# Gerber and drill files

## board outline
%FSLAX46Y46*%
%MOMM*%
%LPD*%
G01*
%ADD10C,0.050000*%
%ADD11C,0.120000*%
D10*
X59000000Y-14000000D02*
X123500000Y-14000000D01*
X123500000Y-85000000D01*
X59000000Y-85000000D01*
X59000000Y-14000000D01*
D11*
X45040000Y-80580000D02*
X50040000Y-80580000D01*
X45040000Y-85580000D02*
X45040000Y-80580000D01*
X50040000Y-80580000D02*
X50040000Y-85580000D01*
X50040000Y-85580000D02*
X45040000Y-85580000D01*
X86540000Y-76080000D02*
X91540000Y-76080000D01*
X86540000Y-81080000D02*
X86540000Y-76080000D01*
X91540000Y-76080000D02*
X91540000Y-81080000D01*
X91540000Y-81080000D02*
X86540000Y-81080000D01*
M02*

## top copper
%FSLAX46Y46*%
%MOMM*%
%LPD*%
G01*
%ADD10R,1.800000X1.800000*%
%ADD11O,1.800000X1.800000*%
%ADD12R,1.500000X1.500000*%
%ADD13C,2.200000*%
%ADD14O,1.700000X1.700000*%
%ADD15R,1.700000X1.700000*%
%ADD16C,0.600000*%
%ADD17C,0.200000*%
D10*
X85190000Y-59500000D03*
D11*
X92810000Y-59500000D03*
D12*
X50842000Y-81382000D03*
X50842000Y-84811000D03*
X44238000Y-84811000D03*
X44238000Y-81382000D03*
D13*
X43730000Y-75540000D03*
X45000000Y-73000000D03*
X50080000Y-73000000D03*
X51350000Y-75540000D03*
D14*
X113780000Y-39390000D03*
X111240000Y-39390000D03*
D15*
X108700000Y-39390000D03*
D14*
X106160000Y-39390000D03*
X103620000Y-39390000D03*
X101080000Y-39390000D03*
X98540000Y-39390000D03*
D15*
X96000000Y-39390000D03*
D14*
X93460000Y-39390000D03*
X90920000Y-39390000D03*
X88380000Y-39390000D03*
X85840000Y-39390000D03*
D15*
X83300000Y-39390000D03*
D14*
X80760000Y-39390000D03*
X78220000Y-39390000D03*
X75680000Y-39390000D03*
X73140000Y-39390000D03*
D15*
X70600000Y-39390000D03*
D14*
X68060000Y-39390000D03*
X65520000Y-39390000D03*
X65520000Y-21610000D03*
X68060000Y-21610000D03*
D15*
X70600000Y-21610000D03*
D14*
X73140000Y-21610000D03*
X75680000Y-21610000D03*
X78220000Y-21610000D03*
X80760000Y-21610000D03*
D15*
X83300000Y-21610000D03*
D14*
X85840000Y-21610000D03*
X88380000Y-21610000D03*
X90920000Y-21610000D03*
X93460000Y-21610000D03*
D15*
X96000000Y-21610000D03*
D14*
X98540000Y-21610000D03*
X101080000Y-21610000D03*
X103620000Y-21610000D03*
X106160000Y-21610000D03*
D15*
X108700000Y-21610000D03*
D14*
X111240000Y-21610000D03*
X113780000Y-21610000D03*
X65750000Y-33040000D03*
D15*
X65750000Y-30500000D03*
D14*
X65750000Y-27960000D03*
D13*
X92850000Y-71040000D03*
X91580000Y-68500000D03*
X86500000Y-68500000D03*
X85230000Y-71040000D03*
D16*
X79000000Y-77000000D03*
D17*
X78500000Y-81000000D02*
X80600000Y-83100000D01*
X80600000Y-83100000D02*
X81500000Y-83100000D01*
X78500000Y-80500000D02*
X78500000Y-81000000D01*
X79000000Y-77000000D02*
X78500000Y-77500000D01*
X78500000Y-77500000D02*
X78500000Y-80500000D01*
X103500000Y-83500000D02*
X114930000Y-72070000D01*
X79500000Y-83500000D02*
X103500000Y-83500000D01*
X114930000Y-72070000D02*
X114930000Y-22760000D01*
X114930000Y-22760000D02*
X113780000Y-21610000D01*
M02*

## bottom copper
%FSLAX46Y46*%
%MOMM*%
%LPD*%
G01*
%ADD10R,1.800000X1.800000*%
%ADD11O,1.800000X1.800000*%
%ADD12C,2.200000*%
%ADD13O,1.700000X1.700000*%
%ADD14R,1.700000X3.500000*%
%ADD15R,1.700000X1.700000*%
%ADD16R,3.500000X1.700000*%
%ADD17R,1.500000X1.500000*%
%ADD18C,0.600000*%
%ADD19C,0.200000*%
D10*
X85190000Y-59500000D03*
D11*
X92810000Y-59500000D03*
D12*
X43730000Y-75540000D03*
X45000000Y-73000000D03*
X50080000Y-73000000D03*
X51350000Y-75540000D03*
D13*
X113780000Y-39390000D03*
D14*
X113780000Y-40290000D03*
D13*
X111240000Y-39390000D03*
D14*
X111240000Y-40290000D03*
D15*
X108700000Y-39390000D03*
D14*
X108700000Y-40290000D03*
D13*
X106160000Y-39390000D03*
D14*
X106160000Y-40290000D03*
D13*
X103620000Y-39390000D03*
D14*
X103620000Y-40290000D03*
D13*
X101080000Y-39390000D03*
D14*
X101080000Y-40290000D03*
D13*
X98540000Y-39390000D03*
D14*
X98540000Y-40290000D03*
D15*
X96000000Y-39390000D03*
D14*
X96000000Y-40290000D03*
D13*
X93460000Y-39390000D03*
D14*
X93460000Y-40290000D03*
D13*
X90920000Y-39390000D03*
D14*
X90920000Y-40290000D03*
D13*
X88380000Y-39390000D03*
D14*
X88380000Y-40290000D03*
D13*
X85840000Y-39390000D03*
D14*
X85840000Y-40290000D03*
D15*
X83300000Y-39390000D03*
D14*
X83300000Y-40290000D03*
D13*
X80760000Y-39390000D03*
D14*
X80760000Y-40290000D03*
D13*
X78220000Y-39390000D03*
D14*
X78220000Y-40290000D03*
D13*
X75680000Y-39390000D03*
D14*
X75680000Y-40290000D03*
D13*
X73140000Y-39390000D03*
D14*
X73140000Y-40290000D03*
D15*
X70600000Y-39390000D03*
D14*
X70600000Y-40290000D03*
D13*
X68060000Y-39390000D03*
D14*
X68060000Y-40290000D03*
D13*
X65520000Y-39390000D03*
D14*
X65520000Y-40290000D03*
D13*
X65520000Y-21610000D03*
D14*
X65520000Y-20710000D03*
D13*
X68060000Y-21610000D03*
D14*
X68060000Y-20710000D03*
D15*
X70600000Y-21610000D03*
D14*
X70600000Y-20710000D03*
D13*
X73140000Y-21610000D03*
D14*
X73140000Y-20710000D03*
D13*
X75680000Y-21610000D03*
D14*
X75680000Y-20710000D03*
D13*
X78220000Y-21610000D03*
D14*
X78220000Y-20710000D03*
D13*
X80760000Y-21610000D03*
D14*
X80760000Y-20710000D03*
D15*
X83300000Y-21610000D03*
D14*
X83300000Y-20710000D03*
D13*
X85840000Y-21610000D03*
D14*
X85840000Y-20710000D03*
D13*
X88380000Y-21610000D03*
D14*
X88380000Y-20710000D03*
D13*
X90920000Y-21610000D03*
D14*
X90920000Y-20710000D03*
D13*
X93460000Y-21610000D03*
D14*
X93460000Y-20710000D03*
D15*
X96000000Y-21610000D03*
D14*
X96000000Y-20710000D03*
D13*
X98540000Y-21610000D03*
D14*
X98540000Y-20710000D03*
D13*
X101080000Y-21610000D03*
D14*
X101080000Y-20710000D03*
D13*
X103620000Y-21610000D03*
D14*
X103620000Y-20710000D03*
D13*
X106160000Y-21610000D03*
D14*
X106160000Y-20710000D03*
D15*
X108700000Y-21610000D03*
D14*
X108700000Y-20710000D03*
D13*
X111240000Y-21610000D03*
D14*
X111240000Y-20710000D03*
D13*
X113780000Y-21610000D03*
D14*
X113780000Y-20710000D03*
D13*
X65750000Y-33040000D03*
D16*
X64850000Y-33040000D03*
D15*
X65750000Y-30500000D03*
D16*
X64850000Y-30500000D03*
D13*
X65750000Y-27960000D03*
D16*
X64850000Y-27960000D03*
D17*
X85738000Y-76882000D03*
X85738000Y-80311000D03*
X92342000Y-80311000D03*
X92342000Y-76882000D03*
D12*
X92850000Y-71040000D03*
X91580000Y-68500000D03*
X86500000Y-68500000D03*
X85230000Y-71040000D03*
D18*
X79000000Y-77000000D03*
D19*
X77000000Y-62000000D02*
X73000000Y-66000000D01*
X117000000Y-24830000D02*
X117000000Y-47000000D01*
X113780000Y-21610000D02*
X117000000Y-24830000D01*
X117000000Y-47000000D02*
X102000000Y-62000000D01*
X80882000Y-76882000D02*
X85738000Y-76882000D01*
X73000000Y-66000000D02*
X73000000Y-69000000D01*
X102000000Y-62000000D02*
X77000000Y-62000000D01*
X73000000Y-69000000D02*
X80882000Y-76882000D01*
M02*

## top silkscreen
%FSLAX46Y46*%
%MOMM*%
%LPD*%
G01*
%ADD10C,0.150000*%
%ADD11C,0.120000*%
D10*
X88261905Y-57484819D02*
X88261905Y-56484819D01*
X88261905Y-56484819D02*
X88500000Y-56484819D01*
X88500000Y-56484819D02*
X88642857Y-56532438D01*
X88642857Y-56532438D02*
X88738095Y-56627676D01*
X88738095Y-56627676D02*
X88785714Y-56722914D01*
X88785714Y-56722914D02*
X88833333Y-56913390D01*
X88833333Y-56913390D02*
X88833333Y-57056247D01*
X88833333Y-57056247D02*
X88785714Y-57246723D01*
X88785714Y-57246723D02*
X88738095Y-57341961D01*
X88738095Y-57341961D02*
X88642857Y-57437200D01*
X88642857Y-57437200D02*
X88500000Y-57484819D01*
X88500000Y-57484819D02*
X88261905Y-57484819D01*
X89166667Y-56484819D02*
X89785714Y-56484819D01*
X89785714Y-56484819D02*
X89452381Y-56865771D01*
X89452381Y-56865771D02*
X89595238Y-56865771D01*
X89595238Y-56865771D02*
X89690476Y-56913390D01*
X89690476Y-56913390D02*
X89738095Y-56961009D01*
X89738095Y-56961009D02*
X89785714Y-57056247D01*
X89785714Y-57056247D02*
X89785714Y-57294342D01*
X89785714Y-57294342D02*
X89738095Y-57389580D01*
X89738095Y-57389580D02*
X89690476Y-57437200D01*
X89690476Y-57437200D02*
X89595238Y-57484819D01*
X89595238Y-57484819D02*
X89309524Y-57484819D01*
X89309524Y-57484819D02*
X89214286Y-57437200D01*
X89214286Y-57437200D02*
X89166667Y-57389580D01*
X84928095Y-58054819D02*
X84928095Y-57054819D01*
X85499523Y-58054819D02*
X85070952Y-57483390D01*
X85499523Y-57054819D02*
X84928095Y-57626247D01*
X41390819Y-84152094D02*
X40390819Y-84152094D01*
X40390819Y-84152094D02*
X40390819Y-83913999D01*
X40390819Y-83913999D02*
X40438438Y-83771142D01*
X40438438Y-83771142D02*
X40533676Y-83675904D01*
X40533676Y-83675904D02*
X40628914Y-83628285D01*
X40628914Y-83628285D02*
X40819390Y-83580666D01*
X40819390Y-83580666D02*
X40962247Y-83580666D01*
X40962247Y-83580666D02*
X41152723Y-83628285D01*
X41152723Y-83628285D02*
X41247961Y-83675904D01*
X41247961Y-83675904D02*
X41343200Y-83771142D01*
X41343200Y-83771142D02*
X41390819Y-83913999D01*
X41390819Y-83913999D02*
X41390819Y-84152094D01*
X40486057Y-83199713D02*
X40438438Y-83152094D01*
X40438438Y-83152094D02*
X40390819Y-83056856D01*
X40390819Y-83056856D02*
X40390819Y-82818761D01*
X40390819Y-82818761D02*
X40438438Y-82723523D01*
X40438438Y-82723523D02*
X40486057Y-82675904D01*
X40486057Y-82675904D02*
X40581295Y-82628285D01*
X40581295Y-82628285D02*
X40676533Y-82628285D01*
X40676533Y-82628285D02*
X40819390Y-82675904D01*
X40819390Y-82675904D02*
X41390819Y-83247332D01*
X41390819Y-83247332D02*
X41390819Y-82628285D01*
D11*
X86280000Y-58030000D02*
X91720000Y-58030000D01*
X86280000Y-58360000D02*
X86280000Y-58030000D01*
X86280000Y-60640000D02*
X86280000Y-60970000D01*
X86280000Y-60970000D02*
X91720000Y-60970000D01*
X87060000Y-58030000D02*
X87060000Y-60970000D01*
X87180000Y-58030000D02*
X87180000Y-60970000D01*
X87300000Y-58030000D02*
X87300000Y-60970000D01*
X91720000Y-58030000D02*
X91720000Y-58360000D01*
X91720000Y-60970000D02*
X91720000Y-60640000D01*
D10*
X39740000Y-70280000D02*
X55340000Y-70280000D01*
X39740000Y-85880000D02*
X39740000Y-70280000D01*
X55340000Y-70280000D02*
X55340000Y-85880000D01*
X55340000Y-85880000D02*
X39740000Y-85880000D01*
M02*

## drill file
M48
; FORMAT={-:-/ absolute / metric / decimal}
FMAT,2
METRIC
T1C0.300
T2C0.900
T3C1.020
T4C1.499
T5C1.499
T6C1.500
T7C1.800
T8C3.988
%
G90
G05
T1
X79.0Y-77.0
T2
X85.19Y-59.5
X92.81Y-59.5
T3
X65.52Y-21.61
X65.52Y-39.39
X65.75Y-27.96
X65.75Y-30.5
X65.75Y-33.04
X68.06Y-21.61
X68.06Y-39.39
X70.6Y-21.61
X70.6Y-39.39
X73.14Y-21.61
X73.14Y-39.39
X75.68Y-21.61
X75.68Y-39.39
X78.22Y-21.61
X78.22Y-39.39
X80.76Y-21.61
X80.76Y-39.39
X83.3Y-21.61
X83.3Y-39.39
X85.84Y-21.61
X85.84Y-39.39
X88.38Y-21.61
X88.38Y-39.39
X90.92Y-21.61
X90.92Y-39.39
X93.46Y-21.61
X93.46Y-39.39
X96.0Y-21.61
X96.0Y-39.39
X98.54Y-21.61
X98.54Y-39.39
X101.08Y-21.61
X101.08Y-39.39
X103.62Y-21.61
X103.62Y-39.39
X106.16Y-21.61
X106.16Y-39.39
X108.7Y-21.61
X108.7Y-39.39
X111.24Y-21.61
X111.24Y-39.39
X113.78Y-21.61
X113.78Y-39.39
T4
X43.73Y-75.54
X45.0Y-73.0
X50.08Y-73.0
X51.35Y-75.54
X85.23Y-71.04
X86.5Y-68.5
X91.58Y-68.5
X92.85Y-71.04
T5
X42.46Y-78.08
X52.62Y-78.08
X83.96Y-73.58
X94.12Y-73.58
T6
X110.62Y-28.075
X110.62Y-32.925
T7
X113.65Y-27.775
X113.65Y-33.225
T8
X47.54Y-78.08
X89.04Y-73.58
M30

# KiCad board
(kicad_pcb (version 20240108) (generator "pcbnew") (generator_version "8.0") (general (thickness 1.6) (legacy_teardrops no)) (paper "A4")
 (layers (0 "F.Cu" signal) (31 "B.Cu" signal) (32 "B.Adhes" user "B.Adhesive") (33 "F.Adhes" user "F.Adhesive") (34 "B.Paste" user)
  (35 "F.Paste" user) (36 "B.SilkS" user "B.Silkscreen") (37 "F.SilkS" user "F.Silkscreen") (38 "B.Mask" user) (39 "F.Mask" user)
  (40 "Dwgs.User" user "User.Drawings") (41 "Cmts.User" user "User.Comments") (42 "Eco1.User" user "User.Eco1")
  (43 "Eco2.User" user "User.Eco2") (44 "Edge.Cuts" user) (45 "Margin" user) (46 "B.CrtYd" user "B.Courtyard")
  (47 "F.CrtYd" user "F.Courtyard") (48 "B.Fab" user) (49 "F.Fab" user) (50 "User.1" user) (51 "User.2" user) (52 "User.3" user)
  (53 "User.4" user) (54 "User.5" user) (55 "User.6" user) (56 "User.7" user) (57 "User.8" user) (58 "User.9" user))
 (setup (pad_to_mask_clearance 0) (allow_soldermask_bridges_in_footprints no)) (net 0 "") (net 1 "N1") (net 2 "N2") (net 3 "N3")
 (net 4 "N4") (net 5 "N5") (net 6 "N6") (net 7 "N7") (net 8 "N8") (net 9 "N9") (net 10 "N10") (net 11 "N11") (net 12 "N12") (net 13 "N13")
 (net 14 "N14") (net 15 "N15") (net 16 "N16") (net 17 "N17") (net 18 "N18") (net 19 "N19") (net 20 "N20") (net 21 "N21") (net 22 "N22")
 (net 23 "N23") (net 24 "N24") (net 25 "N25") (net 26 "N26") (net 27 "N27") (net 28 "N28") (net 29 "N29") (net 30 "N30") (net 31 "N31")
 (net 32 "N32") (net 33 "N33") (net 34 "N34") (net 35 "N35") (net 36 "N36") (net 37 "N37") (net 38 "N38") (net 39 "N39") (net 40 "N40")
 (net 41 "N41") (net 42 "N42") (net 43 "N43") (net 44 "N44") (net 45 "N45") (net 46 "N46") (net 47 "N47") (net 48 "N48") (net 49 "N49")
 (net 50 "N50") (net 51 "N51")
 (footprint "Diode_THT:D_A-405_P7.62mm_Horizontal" (layer "F.Cu") (at 85.19 59.5)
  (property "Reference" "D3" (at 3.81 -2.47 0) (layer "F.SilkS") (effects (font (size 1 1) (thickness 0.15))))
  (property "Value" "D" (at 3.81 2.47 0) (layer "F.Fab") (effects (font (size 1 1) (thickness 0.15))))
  (fp_line (start 1.09 -1.47) (end 6.53 -1.47) (stroke (width 0.12) (type solid)) (layer "F.SilkS"))
  (fp_line (start 1.09 -1.14) (end 1.09 -1.47) (stroke (width 0.12) (type solid)) (layer "F.SilkS"))
  (fp_line (start 1.09 1.14) (end 1.09 1.47) (stroke (width 0.12) (type solid)) (layer "F.SilkS"))
  (fp_line (start 1.09 1.47) (end 6.53 1.47) (stroke (width 0.12) (type solid)) (layer "F.SilkS"))
  (fp_line (start 1.87 -1.47) (end 1.87 1.47) (stroke (width 0.12) (type solid)) (layer "F.SilkS"))
  (fp_line (start 1.99 -1.47) (end 1.99 1.47) (stroke (width 0.12) (type solid)) (layer "F.SilkS"))
  (fp_line (start 2.11 -1.47) (end 2.11 1.47) (stroke (width 0.12) (type solid)) (layer "F.SilkS"))
  (fp_line (start 6.53 -1.47) (end 6.53 -1.14) (stroke (width 0.12) (type solid)) (layer "F.SilkS"))
  (fp_line (start 6.53 1.47) (end 6.53 1.14) (stroke (width 0.12) (type solid)) (layer "F.SilkS"))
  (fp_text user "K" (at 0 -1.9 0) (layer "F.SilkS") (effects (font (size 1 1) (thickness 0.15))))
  (pad "1" thru_hole rect (at 0 0) (size 1.8 1.8) (drill 0.9) (layers "*.Cu" "*.Mask") (remove_unused_layers no) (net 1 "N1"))
  (pad "2" thru_hole oval (at 7.62 0) (size 1.8 1.8) (drill 0.9) (layers "*.Cu" "*.Mask") (remove_unused_layers no) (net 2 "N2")))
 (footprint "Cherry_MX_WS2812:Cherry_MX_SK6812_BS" (layer "F.Cu") (at 47.54 78.08)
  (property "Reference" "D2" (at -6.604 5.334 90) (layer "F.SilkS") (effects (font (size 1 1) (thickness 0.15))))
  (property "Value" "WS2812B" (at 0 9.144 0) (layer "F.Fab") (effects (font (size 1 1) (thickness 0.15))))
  (fp_line (start -7.8 -7.8) (end 7.8 -7.8) (stroke (width 0.15) (type solid)) (layer "F.SilkS"))
  (fp_line (start -7.8 7.8) (end -7.8 -7.8) (stroke (width 0.15) (type solid)) (layer "F.SilkS"))
  (fp_line (start 7.8 -7.8) (end 7.8 7.8) (stroke (width 0.15) (type solid)) (layer "F.SilkS"))
  (fp_line (start 7.8 7.8) (end -7.8 7.8) (stroke (width 0.15) (type solid)) (layer "F.SilkS"))
  (fp_line (start -2.5 2.5) (end 2.5 2.5) (stroke (width 0.12) (type solid)) (layer "Edge.Cuts"))
  (fp_line (start -2.5 7.5) (end -2.5 2.5) (stroke (width 0.12) (type solid)) (layer "Edge.Cuts"))
  (fp_line (start 2.5 2.5) (end 2.5 7.5) (stroke (width 0.12) (type solid)) (layer "Edge.Cuts"))
  (fp_line (start 2.5 7.5) (end -2.5 7.5) (stroke (width 0.12) (type solid)) (layer "Edge.Cuts"))
  (pad "" np_thru_hole circle (at -5.08 0) (size 1.4986 1.4986) (drill 1.4986) (layers "*.Cu" "*.Mask"))
  (pad "" np_thru_hole circle (at 0 0) (size 3.9878 3.9878) (drill 3.9878) (layers "*.Cu" "*.Mask"))
  (pad "" np_thru_hole circle (at 5.08 0) (size 1.4986 1.4986) (drill 1.4986) (layers "*.Cu" "*.Mask"))
  (pad "1" smd rect (at 3.302 3.302) (size 1.5 1.5) (layers "F.Cu" "F.Paste" "F.Mask") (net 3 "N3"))
  (pad "2" smd rect (at 3.302 6.731) (size 1.5 1.5) (layers "F.Cu" "F.Paste" "F.Mask") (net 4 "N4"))
  (pad "3" smd rect (at -3.302 6.731) (size 1.5 1.5) (layers "F.Cu" "F.Paste" "F.Mask") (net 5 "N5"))
  (pad "4" smd rect (at -3.302 3.302) (size 1.5 1.5) (layers "F.Cu" "F.Paste" "F.Mask") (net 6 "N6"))
  (pad "5" thru_hole circle (at -3.81 -2.54) (size 2.2 2.2) (drill 1.4986) (layers "*.Cu" "*.Mask") (remove_unused_layers no) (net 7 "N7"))
  (pad "5" thru_hole circle (at -2.54 -5.08) (size 2.2 2.2) (drill 1.4986) (layers "*.Cu" "*.Mask") (remove_unused_layers no) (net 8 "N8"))
  (pad "6" thru_hole circle (at 2.54 -5.08) (size 2.2 2.2) (drill 1.4986) (layers "*.Cu" "*.Mask") (remove_unused_layers no) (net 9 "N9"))
  (pad "6" thru_hole circle (at 3.81 -2.54) (size 2.2 2.2) (drill 1.4986) (layers "*.Cu" "*.Mask") (remove_unused_layers no) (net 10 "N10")))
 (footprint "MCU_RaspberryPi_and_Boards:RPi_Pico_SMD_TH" (layer "B.Cu") (at 89.65 30.5 90)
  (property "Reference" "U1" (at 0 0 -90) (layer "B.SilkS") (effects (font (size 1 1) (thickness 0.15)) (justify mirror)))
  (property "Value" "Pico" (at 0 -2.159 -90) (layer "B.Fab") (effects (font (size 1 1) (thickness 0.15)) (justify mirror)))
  (pad "" np_thru_hole oval (at -2.725 24 90) (size 1.8 1.8) (drill 1.8) (layers "*.Cu" "*.Mask"))
  (pad "" np_thru_hole oval (at -2.425 20.97 90) (size 1.5 1.5) (drill 1.5) (layers "*.Cu" "*.Mask"))
  (pad "" np_thru_hole oval (at 2.425 20.97 90) (size 1.5 1.5) (drill 1.5) (layers "*.Cu" "*.Mask"))
  (pad "" np_thru_hole oval (at 2.725 24 90) (size 1.8 1.8) (drill 1.8) (layers "*.Cu" "*.Mask"))
  (pad "1" thru_hole oval (at -8.89 24.13 90) (size 1.7 1.7) (drill 1.02) (layers "*.Cu" "*.Mask") (remove_unused_layers no) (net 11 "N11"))
  (pad "1" smd rect (at -8.89 24.13 90) (size 3.5 1.7) (drill (offset -0.9 0)) (layers "B.Cu" "B.Mask") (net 11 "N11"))
  (pad "2" thru_hole oval (at -8.89 21.59 90) (size 1.7 1.7) (drill 1.02) (layers "*.Cu" "*.Mask") (remove_unused_layers no) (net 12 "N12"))
  (pad "2" smd rect (at -8.89 21.59 90) (size 3.5 1.7) (drill (offset -0.9 0)) (layers "B.Cu" "B.Mask") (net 12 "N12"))
  (pad "3" thru_hole rect (at -8.89 19.05 90) (size 1.7 1.7) (drill 1.02) (layers "*.Cu" "*.Mask") (remove_unused_layers no) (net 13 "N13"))
  (pad "3" smd rect (at -8.89 19.05 90) (size 3.5 1.7) (drill (offset -0.9 0)) (layers "B.Cu" "B.Mask") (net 13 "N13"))
  (pad "4" thru_hole oval (at -8.89 16.51 90) (size 1.7 1.7) (drill 1.02) (layers "*.Cu" "*.Mask") (remove_unused_layers no) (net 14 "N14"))
  (pad "4" smd rect (at -8.89 16.51 90) (size 3.5 1.7) (drill (offset -0.9 0)) (layers "B.Cu" "B.Mask") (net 14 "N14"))
  (pad "5" thru_hole oval (at -8.89 13.97 90) (size 1.7 1.7) (drill 1.02) (layers "*.Cu" "*.Mask") (remove_unused_layers no) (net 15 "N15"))
  (pad "5" smd rect (at -8.89 13.97 90) (size 3.5 1.7) (drill (offset -0.9 0)) (layers "B.Cu" "B.Mask") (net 15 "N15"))
  (pad "6" thru_hole oval (at -8.89 11.43 90) (size 1.7 1.7) (drill 1.02) (layers "*.Cu" "*.Mask") (remove_unused_layers no) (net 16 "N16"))
  (pad "6" smd rect (at -8.89 11.43 90) (size 3.5 1.7) (drill (offset -0.9 0)) (layers "B.Cu" "B.Mask") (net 16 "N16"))
  (pad "7" thru_hole oval (at -8.89 8.89 90) (size 1.7 1.7) (drill 1.02) (layers "*.Cu" "*.Mask") (remove_unused_layers no) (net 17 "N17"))
  (pad "7" smd rect (at -8.89 8.89 90) (size 3.5 1.7) (drill (offset -0.9 0)) (layers "B.Cu" "B.Mask") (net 17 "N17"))
  (pad "8" thru_hole rect (at -8.89 6.35 90) (size 1.7 1.7) (drill 1.02) (layers "*.Cu" "*.Mask") (remove_unused_layers no) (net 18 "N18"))
  (pad "8" smd rect (at -8.89 6.35 90) (size 3.5 1.7) (drill (offset -0.9 0)) (layers "B.Cu" "B.Mask") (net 18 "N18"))
  (pad "9" thru_hole oval (at -8.89 3.81 90) (size 1.7 1.7) (drill 1.02) (layers "*.Cu" "*.Mask") (remove_unused_layers no) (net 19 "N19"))
  (pad "9" smd rect (at -8.89 3.81 90) (size 3.5 1.7) (drill (offset -0.9 0)) (layers "B.Cu" "B.Mask") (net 19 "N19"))
  (pad "10" thru_hole oval (at -8.89 1.27 90) (size 1.7 1.7) (drill 1.02) (layers "*.Cu" "*.Mask") (remove_unused_layers no) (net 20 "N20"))
  (pad "10" smd rect (at -8.89 1.27 90) (size 3.5 1.7) (drill (offset -0.9 0)) (layers "B.Cu" "B.Mask") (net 20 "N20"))
  (pad "11" thru_hole oval (at -8.89 -1.27 90) (size 1.7 1.7) (drill 1.02) (layers "*.Cu" "*.Mask") (remove_unused_layers no) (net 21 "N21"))
  (pad "11" smd rect (at -8.89 -1.27 90) (size 3.5 1.7) (drill (offset -0.9 0)) (layers "B.Cu" "B.Mask") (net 21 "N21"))
  (pad "12" thru_hole oval (at -8.89 -3.81 90) (size 1.7 1.7) (drill 1.02) (layers "*.Cu" "*.Mask") (remove_unused_layers no) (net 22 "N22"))
  (pad "12" smd rect (at -8.89 -3.81 90) (size 3.5 1.7) (drill (offset -0.9 0)) (layers "B.Cu" "B.Mask") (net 22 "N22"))
  (pad "13" thru_hole rect (at -8.89 -6.35 90) (size 1.7 1.7) (drill 1.02) (layers "*.Cu" "*.Mask") (remove_unused_layers no) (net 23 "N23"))
  (pad "13" smd rect (at -8.89 -6.35 90) (size 3.5 1.7) (drill (offset -0.9 0)) (layers "B.Cu" "B.Mask") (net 23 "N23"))
  (pad "14" thru_hole oval (at -8.89 -8.89 90) (size 1.7 1.7) (drill 1.02) (layers "*.Cu" "*.Mask") (remove_unused_layers no) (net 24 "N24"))
  (pad "14" smd rect (at -8.89 -8.89 90) (size 3.5 1.7) (drill (offset -0.9 0)) (layers "B.Cu" "B.Mask") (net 24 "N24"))
  (pad "15" thru_hole oval (at -8.89 -11.43 90) (size 1.7 1.7) (drill 1.02) (layers "*.Cu" "*.Mask") (remove_unused_layers no)
   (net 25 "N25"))
  (pad "15" smd rect (at -8.89 -11.43 90) (size 3.5 1.7) (drill (offset -0.9 0)) (layers "B.Cu" "B.Mask") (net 25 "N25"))
  (pad "16" thru_hole oval (at -8.89 -13.97 90) (size 1.7 1.7) (drill 1.02) (layers "*.Cu" "*.Mask") (remove_unused_layers no)
   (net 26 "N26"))
  (pad "16" smd rect (at -8.89 -13.97 90) (size 3.5 1.7) (drill (offset -0.9 0)) (layers "B.Cu" "B.Mask") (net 26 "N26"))
  (pad "17" thru_hole oval (at -8.89 -16.51 90) (size 1.7 1.7) (drill 1.02) (layers "*.Cu" "*.Mask") (remove_unused_layers no)
   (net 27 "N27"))
  (pad "17" smd rect (at -8.89 -16.51 90) (size 3.5 1.7) (drill (offset -0.9 0)) (layers "B.Cu" "B.Mask") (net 27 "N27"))
  (pad "18" thru_hole rect (at -8.89 -19.05 90) (size 1.7 1.7) (drill 1.02) (layers "*.Cu" "*.Mask") (remove_unused_layers no)
   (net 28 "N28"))
  (pad "18" smd rect (at -8.89 -19.05 90) (size 3.5 1.7) (drill (offset -0.9 0)) (layers "B.Cu" "B.Mask") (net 28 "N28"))
  (pad "19" thru_hole oval (at -8.89 -21.59 90) (size 1.7 1.7) (drill 1.02) (layers "*.Cu" "*.Mask") (remove_unused_layers no)
   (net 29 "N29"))
  (pad "19" smd rect (at -8.89 -21.59 90) (size 3.5 1.7) (drill (offset -0.9 0)) (layers "B.Cu" "B.Mask") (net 29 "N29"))
  (pad "20" thru_hole oval (at -8.89 -24.13 90) (size 1.7 1.7) (drill 1.02) (layers "*.Cu" "*.Mask") (remove_unused_layers no)
   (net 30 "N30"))
  (pad "20" smd rect (at -8.89 -24.13 90) (size 3.5 1.7) (drill (offset -0.9 0)) (layers "B.Cu" "B.Mask") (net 30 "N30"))
  (pad "21" thru_hole oval (at 8.89 -24.13 90) (size 1.7 1.7) (drill 1.02) (layers "*.Cu" "*.Mask") (remove_unused_layers no) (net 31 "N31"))
  (pad "21" smd rect (at 8.89 -24.13 90) (size 3.5 1.7) (drill (offset 0.9 0)) (layers "B.Cu" "B.Mask") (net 31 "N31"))
  (pad "22" thru_hole oval (at 8.89 -21.59 90) (size 1.7 1.7) (drill 1.02) (layers "*.Cu" "*.Mask") (remove_unused_layers no) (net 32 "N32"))
  (pad "22" smd rect (at 8.89 -21.59 90) (size 3.5 1.7) (drill (offset 0.9 0)) (layers "B.Cu" "B.Mask") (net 32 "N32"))
  (pad "23" thru_hole rect (at 8.89 -19.05 90) (size 1.7 1.7) (drill 1.02) (layers "*.Cu" "*.Mask") (remove_unused_layers no) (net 5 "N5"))
  (pad "23" smd rect (at 8.89 -19.05 90) (size 3.5 1.7) (drill (offset 0.9 0)) (layers "B.Cu" "B.Mask") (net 5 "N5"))
  (pad "24" thru_hole oval (at 8.89 -16.51 90) (size 1.7 1.7) (drill 1.02) (layers "*.Cu" "*.Mask") (remove_unused_layers no) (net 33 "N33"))
  (pad "24" smd rect (at 8.89 -16.51 90) (size 3.5 1.7) (drill (offset 0.9 0)) (layers "B.Cu" "B.Mask") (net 33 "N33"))
  (pad "25" thru_hole oval (at 8.89 -13.97 90) (size 1.7 1.7) (drill 1.02) (layers "*.Cu" "*.Mask") (remove_unused_layers no) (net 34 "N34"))
  (pad "25" smd rect (at 8.89 -13.97 90) (size 3.5 1.7) (drill (offset 0.9 0)) (layers "B.Cu" "B.Mask") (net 34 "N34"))
  (pad "26" thru_hole oval (at 8.89 -11.43 90) (size 1.7 1.7) (drill 1.02) (layers "*.Cu" "*.Mask") (remove_unused_layers no) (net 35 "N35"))
  (pad "26" smd rect (at 8.89 -11.43 90) (size 3.5 1.7) (drill (offset 0.9 0)) (layers "B.Cu" "B.Mask") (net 35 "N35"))
  (pad "27" thru_hole oval (at 8.89 -8.89 90) (size 1.7 1.7) (drill 1.02) (layers "*.Cu" "*.Mask") (remove_unused_layers no) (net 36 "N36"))
  (pad "27" smd rect (at 8.89 -8.89 90) (size 3.5 1.7) (drill (offset 0.9 0)) (layers "B.Cu" "B.Mask") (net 36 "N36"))
  (pad "28" thru_hole rect (at 8.89 -6.35 90) (size 1.7 1.7) (drill 1.02) (layers "*.Cu" "*.Mask") (remove_unused_layers no) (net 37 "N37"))
  (pad "28" smd rect (at 8.89 -6.35 90) (size 3.5 1.7) (drill (offset 0.9 0)) (layers "B.Cu" "B.Mask") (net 37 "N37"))
  (pad "29" thru_hole oval (at 8.89 -3.81 90) (size 1.7 1.7) (drill 1.02) (layers "*.Cu" "*.Mask") (remove_unused_layers no) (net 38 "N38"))
  (pad "29" smd rect (at 8.89 -3.81 90) (size 3.5 1.7) (drill (offset 0.9 0)) (layers "B.Cu" "B.Mask") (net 38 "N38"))
  (pad "30" thru_hole oval (at 8.89 -1.27 90) (size 1.7 1.7) (drill 1.02) (layers "*.Cu" "*.Mask") (remove_unused_layers no) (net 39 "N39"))
  (pad "30" smd rect (at 8.89 -1.27 90) (size 3.5 1.7) (drill (offset 0.9 0)) (layers "B.Cu" "B.Mask") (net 39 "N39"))
  (pad "31" thru_hole oval (at 8.89 1.27 90) (size 1.7 1.7) (drill 1.02) (layers "*.Cu" "*.Mask") (remove_unused_layers no) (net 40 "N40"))
  (pad "31" smd rect (at 8.89 1.27 90) (size 3.5 1.7) (drill (offset 0.9 0)) (layers "B.Cu" "B.Mask") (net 40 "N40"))
  (pad "32" thru_hole oval (at 8.89 3.81 90) (size 1.7 1.7) (drill 1.02) (layers "*.Cu" "*.Mask") (remove_unused_layers no) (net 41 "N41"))
  (pad "32" smd rect (at 8.89 3.81 90) (size 3.5 1.7) (drill (offset 0.9 0)) (layers "B.Cu" "B.Mask") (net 41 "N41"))
  (pad "33" thru_hole rect (at 8.89 6.35 90) (size 1.7 1.7) (drill 1.02) (layers "*.Cu" "*.Mask") (remove_unused_layers no) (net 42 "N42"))
  (pad "33" smd rect (at 8.89 6.35 90) (size 3.5 1.7) (drill (offset 0.9 0)) (layers "B.Cu" "B.Mask") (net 42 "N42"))
  (pad "34" thru_hole oval (at 8.89 8.89 90) (size 1.7 1.7) (drill 1.02) (layers "*.Cu" "*.Mask") (remove_unused_layers no) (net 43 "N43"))
  (pad "34" smd rect (at 8.89 8.89 90) (size 3.5 1.7) (drill (offset 0.9 0)) (layers "B.Cu" "B.Mask") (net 43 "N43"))
  (pad "35" thru_hole oval (at 8.89 11.43 90) (size 1.7 1.7) (drill 1.02) (layers "*.Cu" "*.Mask") (remove_unused_layers no) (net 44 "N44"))
  (pad "35" smd rect (at 8.89 11.43 90) (size 3.5 1.7) (drill (offset 0.9 0)) (layers "B.Cu" "B.Mask") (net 44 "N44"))
  (pad "36" thru_hole oval (at 8.89 13.97 90) (size 1.7 1.7) (drill 1.02) (layers "*.Cu" "*.Mask") (remove_unused_layers no) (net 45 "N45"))
  (pad "36" smd rect (at 8.89 13.97 90) (size 3.5 1.7) (drill (offset 0.9 0)) (layers "B.Cu" "B.Mask") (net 45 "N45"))
  (pad "37" thru_hole oval (at 8.89 16.51 90) (size 1.7 1.7) (drill 1.02) (layers "*.Cu" "*.Mask") (remove_unused_layers no) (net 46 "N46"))
  (pad "37" smd rect (at 8.89 16.51 90) (size 3.5 1.7) (drill (offset 0.9 0)) (layers "B.Cu" "B.Mask") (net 46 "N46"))
  (pad "38" thru_hole rect (at 8.89 19.05 90) (size 1.7 1.7) (drill 1.02) (layers "*.Cu" "*.Mask") (remove_unused_layers no) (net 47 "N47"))
  (pad "38" smd rect (at 8.89 19.05 90) (size 3.5 1.7) (drill (offset 0.9 0)) (layers "B.Cu" "B.Mask") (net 47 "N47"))
  (pad "39" thru_hole oval (at 8.89 21.59 90) (size 1.7 1.7) (drill 1.02) (layers "*.Cu" "*.Mask") (remove_unused_layers no) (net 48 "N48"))
  (pad "39" smd rect (at 8.89 21.59 90) (size 3.5 1.7) (drill (offset 0.9 0)) (layers "B.Cu" "B.Mask") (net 48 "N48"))
  (pad "40" thru_hole oval (at 8.89 24.13 90) (size 1.7 1.7) (drill 1.02) (layers "*.Cu" "*.Mask") (remove_unused_layers no) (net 3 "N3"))
  (pad "40" smd rect (at 8.89 24.13 90) (size 3.5 1.7) (drill (offset 0.9 0)) (layers "B.Cu" "B.Mask") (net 3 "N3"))
  (pad "41" thru_hole oval (at -2.54 -23.9 90) (size 1.7 1.7) (drill 1.02) (layers "*.Cu" "*.Mask") (remove_unused_layers no) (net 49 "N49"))
  (pad "41" smd rect (at -2.54 -23.9) (size 3.5 1.7) (drill (offset -0.9 0)) (layers "B.Cu" "B.Mask") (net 49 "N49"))
  (pad "42" thru_hole rect (at 0 -23.9 90) (size 1.7 1.7) (drill 1.02) (layers "*.Cu" "*.Mask") (remove_unused_layers no) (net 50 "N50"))
  (pad "42" smd rect (at 0 -23.9) (size 3.5 1.7) (drill (offset -0.9 0)) (layers "B.Cu" "B.Mask") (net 50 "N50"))
  (pad "43" thru_hole oval (at 2.54 -23.9 90) (size 1.7 1.7) (drill 1.02) (layers "*.Cu" "*.Mask") (remove_unused_layers no) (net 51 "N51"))
  (pad "43" smd rect (at 2.54 -23.9) (size 3.5 1.7) (drill (offset -0.9 0)) (layers "B.Cu" "B.Mask") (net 51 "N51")))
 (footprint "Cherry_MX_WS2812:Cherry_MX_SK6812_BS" (layer "B.Cu") (at 89.04 73.58 180)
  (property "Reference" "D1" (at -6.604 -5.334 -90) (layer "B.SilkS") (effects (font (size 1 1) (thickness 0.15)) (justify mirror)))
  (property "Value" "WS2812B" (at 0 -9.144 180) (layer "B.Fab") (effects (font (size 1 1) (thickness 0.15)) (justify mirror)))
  (fp_line (start 2.5 -2.5) (end -2.5 -2.5) (stroke (width 0.12) (type solid)) (layer "Edge.Cuts"))
  (fp_line (start 2.5 -7.5) (end 2.5 -2.5) (stroke (width 0.12) (type solid)) (layer "Edge.Cuts"))
  (fp_line (start -2.5 -2.5) (end -2.5 -7.5) (stroke (width 0.12) (type solid)) (layer "Edge.Cuts"))
  (fp_line (start -2.5 -7.5) (end 2.5 -7.5) (stroke (width 0.12) (type solid)) (layer "Edge.Cuts"))
  (pad "" np_thru_hole circle (at -5.08 0 180) (size 1.4986 1.4986) (drill 1.4986) (layers "*.Cu" "*.Mask"))
  (pad "" np_thru_hole circle (at 0 0 180) (size 3.9878 3.9878) (drill 3.9878) (layers "*.Cu" "*.Mask"))
  (pad "" np_thru_hole circle (at 5.08 0 180) (size 1.4986 1.4986) (drill 1.4986) (layers "*.Cu" "*.Mask"))
  (pad "1" smd rect (at 3.302 -3.302 180) (size 1.5 1.5) (layers "B.Cu" "B.Paste" "B.Mask") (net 3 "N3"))
  (pad "2" smd rect (at 3.302 -6.731 180) (size 1.5 1.5) (layers "B.Cu" "B.Paste" "B.Mask") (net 6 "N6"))
  (pad "3" smd rect (at -3.302 -6.731 180) (size 1.5 1.5) (layers "B.Cu" "B.Paste" "B.Mask") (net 5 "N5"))
  (pad "4" smd rect (at -3.302 -3.302 180) (size 1.5 1.5) (layers "B.Cu" "B.Paste" "B.Mask") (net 41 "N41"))
  (pad "5" thru_hole circle (at -3.81 2.54 180) (size 2.2 2.2) (drill 1.4986) (layers "*.Cu" "*.Mask") (remove_unused_layers no)
   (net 38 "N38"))
  (pad "5" thru_hole circle (at -2.54 5.08 180) (size 2.2 2.2) (drill 1.4986) (layers "*.Cu" "*.Mask") (remove_unused_layers no)
   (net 38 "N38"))
  (pad "6" thru_hole circle (at 2.54 5.08 180) (size 2.2 2.2) (drill 1.4986) (layers "*.Cu" "*.Mask") (remove_unused_layers no)
   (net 47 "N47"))
  (pad "6" thru_hole circle (at 3.81 2.54 180) (size 2.2 2.2) (drill 1.4986) (layers "*.Cu" "*.Mask") (remove_unused_layers no)
   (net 47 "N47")))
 (gr_rect (start 59 14) (end 123.5 85) (stroke (width 0.05) (type default)) (fill none) (layer "Edge.Cuts"))
 (segment (start 78.5 81) (end 80.6 83.1) (width 0.2) (layer "F.Cu") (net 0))
 (segment (start 80.6 83.1) (end 81.5 83.1) (width 0.2) (layer "F.Cu") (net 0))
 (segment (start 78.5 80.5) (end 78.5 81) (width 0.2) (layer "F.Cu") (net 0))
 (segment (start 79 77) (end 78.5 77.5) (width 0.2) (layer "F.Cu") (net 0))
 (segment (start 78.5 77.5) (end 78.5 80.5) (width 0.2) (layer "F.Cu") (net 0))
 (via (at 79 77) (size 0.6) (drill 0.3) (layers "F.Cu" "B.Cu") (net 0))
 (segment (start 103.5 83.5) (end 114.93 72.07) (width 0.2) (layer "F.Cu") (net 3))
 (segment (start 79.5 83.5) (end 103.5 83.5) (width 0.2) (layer "F.Cu") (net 3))
 (segment (start 114.93 72.07) (end 114.93 22.76) (width 0.2) (layer "F.Cu") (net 3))
 (segment (start 114.93 22.76) (end 113.78 21.61) (width 0.2) (layer "F.Cu") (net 3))
 (segment (start 77 62) (end 73 66) (width 0.2) (layer "B.Cu") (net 3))
 (segment (start 117 24.83) (end 117 47) (width 0.2) (layer "B.Cu") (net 3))
 (segment (start 113.78 21.61) (end 117 24.83) (width 0.2) (layer "B.Cu") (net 3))
 (segment (start 117 47) (end 102 62) (width 0.2) (layer "B.Cu") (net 3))
 (segment (start 80.882 76.882) (end 85.738 76.882) (width 0.2) (layer "B.Cu") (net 3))
 (segment (start 73 66) (end 73 69) (width 0.2) (layer "B.Cu") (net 3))
 (segment (start 102 62) (end 77 62) (width 0.2) (layer "B.Cu") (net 3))
 (segment (start 73 69) (end 80.882 76.882) (width 0.2) (layer "B.Cu") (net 3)))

